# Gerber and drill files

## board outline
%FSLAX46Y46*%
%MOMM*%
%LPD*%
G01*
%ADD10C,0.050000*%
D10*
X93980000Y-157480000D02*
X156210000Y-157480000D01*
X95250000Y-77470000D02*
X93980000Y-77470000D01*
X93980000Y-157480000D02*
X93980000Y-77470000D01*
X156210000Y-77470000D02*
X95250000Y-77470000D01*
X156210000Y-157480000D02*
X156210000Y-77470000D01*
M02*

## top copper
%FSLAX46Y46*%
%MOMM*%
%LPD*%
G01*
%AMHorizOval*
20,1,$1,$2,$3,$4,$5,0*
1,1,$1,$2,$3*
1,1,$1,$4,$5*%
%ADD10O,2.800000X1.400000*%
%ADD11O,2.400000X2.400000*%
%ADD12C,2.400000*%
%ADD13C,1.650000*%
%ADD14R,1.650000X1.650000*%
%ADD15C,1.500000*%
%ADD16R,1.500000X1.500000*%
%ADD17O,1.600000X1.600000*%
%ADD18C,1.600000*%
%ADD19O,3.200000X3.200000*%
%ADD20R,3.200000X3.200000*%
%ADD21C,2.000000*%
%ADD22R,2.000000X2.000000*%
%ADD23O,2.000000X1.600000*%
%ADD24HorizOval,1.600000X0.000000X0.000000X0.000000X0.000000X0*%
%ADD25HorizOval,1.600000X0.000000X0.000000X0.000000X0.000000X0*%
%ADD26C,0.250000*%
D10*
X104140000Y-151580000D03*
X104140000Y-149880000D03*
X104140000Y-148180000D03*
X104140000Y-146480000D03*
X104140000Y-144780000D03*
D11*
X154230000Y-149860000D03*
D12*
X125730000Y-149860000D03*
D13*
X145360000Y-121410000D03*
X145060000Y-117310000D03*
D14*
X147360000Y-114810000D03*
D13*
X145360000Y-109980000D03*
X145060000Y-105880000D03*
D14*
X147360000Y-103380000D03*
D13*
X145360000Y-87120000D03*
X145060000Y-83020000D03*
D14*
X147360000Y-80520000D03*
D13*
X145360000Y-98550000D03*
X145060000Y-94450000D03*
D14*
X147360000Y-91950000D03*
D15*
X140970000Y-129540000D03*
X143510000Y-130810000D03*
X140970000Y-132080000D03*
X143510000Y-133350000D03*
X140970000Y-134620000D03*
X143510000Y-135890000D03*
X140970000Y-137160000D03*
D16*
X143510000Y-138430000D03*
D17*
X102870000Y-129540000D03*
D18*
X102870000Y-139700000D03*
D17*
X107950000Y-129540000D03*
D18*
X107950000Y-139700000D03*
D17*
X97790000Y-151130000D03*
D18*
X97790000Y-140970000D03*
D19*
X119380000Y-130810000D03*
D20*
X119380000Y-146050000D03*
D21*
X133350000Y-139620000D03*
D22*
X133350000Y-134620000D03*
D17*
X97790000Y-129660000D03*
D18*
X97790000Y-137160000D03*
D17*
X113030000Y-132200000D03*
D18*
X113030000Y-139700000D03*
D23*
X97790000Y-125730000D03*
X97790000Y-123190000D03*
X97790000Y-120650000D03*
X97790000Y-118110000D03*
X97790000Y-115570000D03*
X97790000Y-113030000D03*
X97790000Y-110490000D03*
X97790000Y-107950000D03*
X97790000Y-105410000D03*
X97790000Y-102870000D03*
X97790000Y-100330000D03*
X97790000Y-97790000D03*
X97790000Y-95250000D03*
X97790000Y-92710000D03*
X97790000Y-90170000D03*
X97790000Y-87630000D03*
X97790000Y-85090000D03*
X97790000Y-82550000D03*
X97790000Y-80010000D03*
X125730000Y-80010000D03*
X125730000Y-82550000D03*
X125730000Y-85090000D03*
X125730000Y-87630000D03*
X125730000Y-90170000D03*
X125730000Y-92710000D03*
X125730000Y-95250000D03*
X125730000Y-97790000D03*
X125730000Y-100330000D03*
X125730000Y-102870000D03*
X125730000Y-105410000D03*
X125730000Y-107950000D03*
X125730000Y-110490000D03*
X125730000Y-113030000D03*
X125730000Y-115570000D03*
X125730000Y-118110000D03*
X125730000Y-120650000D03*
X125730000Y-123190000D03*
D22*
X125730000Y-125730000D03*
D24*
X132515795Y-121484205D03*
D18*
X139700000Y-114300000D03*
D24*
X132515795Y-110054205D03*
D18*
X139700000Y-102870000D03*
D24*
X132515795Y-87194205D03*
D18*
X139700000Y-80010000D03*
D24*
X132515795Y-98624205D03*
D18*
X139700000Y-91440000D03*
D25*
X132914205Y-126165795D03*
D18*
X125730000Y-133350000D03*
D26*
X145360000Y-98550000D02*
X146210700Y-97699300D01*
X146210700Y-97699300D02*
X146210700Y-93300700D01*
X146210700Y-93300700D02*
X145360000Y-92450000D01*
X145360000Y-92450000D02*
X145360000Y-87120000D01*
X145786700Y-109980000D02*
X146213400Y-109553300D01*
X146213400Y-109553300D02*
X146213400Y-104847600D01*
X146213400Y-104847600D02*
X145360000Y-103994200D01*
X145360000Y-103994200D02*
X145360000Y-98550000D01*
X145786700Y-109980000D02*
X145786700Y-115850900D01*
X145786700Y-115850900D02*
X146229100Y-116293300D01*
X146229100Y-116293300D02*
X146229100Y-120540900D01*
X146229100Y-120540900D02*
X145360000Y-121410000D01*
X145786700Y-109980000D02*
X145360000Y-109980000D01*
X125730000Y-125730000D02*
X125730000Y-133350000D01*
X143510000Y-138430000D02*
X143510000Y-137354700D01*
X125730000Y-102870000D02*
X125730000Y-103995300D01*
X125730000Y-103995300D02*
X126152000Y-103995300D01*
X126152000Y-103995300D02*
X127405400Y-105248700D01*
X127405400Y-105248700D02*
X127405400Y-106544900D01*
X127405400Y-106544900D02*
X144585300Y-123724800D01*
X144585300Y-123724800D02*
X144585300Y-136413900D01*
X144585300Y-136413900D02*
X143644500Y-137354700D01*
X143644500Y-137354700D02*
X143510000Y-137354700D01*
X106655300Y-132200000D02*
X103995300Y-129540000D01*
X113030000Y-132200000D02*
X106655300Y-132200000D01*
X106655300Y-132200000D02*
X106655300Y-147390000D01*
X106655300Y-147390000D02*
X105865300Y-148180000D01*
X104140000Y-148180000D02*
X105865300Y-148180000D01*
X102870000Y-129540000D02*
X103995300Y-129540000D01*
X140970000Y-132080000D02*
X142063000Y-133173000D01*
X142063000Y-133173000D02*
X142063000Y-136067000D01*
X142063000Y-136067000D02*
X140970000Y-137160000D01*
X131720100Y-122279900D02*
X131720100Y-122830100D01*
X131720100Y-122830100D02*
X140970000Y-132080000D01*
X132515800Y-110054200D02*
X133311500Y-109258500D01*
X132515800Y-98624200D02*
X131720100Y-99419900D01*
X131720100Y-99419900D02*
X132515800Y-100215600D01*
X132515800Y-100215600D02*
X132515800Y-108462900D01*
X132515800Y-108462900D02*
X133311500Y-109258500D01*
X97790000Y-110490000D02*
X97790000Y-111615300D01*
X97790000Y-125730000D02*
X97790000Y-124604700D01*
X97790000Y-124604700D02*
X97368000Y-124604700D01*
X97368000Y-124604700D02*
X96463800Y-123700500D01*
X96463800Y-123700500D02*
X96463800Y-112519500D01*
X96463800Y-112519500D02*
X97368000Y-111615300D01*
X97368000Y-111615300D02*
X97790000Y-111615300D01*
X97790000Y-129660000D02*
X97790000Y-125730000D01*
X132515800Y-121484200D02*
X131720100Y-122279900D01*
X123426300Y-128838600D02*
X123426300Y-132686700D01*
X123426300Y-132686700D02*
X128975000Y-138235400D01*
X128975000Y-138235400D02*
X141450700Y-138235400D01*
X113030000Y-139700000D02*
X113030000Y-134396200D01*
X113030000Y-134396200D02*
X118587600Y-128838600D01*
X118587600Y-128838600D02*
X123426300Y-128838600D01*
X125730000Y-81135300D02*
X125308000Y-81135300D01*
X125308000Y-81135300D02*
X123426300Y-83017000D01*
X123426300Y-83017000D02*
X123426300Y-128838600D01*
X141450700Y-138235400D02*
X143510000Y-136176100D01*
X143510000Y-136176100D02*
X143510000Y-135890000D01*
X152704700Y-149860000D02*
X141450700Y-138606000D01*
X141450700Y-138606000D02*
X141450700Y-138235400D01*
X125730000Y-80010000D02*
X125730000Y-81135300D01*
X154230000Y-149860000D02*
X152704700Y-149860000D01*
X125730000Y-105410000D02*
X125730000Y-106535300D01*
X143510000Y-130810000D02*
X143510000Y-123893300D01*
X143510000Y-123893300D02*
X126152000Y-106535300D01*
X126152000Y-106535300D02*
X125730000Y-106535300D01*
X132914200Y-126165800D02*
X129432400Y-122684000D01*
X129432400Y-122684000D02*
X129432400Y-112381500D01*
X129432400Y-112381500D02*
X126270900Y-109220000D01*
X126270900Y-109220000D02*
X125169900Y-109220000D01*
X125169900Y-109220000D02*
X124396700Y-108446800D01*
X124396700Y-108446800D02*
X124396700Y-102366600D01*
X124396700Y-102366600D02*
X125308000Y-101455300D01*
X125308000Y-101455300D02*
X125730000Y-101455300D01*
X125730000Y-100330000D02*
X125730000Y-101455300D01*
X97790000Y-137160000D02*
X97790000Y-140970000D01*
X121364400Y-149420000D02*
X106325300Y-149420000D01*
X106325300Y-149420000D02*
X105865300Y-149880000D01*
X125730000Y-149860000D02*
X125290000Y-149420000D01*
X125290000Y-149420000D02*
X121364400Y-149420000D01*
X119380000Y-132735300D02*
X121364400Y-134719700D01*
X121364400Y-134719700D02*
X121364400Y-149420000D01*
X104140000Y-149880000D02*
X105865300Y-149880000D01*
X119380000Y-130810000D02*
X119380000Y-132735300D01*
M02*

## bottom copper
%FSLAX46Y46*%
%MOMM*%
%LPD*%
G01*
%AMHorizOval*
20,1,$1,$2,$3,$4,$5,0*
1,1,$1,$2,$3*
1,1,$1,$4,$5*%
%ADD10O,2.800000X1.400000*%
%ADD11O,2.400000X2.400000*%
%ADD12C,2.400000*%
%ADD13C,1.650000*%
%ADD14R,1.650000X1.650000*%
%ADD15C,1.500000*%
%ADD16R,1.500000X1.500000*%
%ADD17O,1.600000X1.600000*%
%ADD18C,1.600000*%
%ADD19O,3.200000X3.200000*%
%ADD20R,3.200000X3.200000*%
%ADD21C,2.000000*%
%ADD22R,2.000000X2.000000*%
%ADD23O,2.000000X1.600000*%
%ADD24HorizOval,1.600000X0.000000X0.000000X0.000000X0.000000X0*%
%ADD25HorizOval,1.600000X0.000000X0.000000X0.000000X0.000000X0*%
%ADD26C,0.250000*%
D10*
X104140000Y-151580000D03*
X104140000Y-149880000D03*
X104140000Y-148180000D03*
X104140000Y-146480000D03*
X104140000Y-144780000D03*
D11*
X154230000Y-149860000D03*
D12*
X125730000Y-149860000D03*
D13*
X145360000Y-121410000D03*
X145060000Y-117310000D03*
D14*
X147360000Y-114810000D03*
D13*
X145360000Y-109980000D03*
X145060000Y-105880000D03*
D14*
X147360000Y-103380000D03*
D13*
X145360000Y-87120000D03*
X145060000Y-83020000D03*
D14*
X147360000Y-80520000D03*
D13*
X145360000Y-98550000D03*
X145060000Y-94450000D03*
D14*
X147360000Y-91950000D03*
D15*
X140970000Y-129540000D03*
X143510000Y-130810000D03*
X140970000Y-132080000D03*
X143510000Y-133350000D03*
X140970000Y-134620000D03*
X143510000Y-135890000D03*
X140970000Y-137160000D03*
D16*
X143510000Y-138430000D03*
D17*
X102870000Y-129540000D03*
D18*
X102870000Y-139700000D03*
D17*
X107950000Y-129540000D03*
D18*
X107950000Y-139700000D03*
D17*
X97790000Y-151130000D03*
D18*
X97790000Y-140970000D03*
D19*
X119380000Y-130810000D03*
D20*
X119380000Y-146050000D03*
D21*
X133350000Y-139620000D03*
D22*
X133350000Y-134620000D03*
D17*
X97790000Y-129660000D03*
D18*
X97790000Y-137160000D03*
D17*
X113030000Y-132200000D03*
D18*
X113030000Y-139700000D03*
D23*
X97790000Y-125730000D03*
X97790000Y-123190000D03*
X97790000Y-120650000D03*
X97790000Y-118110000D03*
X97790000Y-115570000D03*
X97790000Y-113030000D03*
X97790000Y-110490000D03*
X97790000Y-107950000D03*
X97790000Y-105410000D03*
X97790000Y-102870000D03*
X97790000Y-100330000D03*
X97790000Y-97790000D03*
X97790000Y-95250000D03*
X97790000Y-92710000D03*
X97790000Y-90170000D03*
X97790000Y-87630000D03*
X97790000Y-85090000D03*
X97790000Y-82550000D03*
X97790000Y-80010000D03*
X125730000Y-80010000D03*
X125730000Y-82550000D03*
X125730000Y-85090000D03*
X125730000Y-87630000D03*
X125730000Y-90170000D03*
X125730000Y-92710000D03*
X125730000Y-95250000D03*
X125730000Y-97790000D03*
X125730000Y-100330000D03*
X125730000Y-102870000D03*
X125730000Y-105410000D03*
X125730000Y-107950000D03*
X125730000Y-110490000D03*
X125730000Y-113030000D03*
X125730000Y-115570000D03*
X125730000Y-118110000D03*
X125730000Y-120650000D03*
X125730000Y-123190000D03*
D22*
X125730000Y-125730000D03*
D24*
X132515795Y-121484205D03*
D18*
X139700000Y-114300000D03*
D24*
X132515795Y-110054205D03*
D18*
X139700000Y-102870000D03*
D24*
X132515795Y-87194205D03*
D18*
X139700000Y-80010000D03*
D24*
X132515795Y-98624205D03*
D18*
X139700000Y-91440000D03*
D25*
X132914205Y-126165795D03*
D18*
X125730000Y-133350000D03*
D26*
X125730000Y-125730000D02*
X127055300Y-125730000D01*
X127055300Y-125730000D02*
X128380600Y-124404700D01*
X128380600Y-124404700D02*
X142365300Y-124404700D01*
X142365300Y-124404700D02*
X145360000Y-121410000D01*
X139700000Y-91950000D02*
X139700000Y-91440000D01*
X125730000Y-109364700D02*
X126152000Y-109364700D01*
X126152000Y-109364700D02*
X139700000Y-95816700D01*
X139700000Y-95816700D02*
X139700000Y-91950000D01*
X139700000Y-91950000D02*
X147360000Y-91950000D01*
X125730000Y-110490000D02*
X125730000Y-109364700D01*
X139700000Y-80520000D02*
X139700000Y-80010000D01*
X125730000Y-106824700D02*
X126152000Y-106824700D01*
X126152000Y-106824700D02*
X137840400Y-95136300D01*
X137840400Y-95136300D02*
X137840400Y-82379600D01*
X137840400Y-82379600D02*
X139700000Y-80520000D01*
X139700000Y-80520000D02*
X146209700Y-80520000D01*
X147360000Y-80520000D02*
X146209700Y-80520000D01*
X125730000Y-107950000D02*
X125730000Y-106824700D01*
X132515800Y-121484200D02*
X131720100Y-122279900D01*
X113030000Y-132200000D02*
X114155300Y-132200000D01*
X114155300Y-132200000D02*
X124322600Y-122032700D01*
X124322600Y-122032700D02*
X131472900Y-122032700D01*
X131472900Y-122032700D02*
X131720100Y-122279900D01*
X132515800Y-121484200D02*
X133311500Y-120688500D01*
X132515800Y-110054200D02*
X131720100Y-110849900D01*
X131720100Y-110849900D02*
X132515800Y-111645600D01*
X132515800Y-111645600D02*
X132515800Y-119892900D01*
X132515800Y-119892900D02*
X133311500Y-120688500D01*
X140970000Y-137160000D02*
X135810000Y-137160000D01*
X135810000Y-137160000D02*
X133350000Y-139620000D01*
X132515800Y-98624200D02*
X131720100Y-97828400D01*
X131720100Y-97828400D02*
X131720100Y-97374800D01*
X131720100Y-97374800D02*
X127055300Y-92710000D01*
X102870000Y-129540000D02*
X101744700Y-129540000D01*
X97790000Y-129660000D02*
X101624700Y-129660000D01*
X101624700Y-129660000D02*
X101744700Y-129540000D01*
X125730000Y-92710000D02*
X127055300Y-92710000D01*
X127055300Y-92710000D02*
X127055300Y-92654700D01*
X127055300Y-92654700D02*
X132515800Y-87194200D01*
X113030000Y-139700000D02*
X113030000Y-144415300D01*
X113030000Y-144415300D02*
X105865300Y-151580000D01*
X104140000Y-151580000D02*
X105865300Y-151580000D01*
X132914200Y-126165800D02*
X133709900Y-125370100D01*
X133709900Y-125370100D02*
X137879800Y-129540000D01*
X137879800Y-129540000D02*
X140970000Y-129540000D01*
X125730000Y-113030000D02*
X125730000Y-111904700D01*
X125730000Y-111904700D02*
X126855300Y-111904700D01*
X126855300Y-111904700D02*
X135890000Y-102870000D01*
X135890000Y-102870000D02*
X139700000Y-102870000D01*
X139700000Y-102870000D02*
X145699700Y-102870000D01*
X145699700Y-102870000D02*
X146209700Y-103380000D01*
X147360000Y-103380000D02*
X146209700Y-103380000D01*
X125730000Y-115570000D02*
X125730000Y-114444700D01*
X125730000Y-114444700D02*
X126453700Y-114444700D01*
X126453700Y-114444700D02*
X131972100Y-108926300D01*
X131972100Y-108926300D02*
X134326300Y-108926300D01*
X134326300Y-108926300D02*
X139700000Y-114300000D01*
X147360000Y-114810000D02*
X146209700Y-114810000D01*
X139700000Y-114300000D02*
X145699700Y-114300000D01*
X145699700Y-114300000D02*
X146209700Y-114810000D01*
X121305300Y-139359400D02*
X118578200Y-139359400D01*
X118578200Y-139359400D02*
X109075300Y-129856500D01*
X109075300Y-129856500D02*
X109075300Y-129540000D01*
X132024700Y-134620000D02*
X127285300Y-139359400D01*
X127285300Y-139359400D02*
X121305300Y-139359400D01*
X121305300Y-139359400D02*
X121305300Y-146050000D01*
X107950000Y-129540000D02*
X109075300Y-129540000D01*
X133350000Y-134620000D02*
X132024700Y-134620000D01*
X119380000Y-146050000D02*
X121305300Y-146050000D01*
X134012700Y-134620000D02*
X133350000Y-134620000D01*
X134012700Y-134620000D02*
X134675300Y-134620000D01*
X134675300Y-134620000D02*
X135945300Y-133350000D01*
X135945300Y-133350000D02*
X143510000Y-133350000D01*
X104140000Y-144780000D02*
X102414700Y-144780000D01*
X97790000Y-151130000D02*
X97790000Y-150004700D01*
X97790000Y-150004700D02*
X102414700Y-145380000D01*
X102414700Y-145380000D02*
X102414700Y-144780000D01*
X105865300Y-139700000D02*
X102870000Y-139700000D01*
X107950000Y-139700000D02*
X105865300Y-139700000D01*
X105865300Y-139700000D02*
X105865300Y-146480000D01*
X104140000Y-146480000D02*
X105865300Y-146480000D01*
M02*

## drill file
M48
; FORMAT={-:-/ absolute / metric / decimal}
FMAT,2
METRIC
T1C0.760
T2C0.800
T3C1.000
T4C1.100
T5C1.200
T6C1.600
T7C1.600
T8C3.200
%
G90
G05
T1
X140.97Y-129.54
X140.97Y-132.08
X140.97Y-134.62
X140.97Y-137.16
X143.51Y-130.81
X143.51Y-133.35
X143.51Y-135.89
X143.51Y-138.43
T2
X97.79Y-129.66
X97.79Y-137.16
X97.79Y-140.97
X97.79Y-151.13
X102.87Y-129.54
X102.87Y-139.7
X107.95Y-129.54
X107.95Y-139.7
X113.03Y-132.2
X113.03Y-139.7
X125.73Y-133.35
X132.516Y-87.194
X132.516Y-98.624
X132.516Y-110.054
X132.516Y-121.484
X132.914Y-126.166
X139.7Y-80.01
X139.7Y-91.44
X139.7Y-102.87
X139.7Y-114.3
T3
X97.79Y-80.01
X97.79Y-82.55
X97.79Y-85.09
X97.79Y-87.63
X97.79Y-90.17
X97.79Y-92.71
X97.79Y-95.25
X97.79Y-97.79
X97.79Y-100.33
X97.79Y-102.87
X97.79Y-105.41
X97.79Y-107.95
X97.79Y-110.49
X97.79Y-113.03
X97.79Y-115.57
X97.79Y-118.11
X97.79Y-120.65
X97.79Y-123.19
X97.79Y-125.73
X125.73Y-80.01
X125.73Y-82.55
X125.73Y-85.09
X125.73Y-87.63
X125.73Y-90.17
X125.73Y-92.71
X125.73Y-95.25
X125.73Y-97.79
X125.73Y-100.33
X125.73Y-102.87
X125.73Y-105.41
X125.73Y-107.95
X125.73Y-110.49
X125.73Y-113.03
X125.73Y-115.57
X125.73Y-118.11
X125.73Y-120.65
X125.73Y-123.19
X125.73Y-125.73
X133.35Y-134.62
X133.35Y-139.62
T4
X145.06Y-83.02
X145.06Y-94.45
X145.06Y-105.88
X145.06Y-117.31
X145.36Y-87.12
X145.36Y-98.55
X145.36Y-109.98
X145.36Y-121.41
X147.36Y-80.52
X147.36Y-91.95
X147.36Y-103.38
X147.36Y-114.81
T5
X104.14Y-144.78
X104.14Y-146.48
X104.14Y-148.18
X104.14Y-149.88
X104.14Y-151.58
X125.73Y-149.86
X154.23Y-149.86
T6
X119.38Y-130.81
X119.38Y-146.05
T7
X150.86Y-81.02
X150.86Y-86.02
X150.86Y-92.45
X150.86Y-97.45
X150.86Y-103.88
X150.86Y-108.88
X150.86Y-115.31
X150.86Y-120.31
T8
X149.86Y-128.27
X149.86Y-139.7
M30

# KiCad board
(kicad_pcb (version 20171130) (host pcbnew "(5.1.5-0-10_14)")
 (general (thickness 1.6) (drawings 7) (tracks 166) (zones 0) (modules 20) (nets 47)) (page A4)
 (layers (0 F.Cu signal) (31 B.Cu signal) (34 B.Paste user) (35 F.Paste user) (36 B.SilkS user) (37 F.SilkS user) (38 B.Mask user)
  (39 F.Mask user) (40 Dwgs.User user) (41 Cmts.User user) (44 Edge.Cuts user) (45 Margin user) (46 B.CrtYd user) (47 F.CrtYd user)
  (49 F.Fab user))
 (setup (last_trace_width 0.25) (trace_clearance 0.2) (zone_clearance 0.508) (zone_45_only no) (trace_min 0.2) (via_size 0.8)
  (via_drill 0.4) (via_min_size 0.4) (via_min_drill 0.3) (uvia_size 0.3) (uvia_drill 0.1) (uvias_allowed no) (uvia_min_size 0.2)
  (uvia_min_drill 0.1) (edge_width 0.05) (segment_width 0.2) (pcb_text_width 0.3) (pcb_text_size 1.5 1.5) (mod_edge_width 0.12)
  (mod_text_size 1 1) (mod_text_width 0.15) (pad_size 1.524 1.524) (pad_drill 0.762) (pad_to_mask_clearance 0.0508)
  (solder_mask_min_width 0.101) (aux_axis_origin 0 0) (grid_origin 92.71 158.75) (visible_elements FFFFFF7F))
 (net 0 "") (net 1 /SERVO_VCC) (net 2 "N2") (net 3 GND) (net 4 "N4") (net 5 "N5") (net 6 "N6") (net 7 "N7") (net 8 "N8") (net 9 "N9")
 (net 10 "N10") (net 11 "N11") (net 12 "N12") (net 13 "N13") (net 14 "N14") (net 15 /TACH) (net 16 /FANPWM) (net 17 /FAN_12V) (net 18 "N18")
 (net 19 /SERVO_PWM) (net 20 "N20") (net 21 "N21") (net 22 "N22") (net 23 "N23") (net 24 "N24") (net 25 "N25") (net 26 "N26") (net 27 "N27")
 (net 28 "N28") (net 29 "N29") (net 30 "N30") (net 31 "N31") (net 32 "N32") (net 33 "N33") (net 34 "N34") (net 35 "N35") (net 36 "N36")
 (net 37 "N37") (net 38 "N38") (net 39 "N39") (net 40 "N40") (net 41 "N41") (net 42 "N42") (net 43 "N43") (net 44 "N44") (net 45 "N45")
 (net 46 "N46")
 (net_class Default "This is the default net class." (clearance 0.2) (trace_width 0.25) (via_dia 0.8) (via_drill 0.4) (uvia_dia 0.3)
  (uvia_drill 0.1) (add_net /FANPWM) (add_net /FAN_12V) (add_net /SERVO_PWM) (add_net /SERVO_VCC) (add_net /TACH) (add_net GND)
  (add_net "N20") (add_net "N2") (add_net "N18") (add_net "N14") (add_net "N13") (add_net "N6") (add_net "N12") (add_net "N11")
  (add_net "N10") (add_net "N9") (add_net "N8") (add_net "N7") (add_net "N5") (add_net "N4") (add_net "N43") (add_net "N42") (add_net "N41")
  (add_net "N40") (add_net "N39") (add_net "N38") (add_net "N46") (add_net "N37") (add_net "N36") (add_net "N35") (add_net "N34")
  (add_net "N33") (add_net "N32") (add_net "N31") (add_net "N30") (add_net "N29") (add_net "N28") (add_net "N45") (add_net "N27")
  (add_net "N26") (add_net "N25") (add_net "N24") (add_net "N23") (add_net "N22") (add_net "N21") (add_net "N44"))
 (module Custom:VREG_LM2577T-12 (layer F.Cu) (at 104.14 144.78 270)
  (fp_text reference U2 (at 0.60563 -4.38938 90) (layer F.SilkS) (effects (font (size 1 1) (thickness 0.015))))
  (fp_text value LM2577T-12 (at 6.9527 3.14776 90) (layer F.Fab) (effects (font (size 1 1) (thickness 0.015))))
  (pad 5 thru_hole oval (at 6.8 0 270) (size 1.4 2.8) (drill 1.2) (layers *.Cu *.Mask) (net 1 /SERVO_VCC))
  (pad 4 thru_hole oval (at 5.1 0 270) (size 1.4 2.8) (drill 1.2) (layers *.Cu *.Mask) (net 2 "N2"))
  (pad 3 thru_hole oval (at 3.4 0 270) (size 1.4 2.8) (drill 1.2) (layers *.Cu *.Mask) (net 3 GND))
  (pad 2 thru_hole oval (at 1.7 0 270) (size 1.4 2.8) (drill 1.2) (layers *.Cu *.Mask) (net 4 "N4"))
  (pad 1 thru_hole oval (at 0 0 270) (size 1.4 2.8) (drill 1.2) (layers *.Cu *.Mask) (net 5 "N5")))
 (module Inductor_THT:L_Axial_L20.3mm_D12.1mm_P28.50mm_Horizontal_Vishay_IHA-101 (layer F.Cu) (at 125.73 149.86)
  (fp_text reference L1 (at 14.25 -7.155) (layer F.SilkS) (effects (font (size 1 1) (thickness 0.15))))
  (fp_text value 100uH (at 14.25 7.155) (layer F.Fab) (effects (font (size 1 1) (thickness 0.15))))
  (pad 2 thru_hole oval (at 28.5 0) (size 2.4 2.4) (drill 1.2) (layers *.Cu *.Mask) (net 1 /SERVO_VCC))
  (pad 1 thru_hole circle (at 0 0) (size 2.4 2.4) (drill 1.2) (layers *.Cu *.Mask) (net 2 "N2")))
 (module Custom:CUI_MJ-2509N (layer F.Cu) (at 149.86 118.11)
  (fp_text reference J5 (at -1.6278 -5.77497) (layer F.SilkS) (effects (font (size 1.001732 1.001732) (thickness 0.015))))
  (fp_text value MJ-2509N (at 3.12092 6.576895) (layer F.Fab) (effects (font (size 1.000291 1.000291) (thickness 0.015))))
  (pad None np_thru_hole circle (at 1 -2.8) (size 1.6 1.6) (drill 1.6) (layers *.Cu *.Mask))
  (pad None np_thru_hole circle (at 1 2.2) (size 1.6 1.6) (drill 1.6) (layers *.Cu *.Mask))
  (pad 3 thru_hole circle (at -4.5 3.3) (size 1.65 1.65) (drill 1.1) (layers *.Cu *.Mask) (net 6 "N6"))
  (pad 2 thru_hole circle (at -4.8 -0.8) (size 1.65 1.65) (drill 1.1) (layers *.Cu *.Mask) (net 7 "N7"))
  (pad 1 thru_hole rect (at -2.5 -3.3) (size 1.65 1.65) (drill 1.1) (layers *.Cu *.Mask) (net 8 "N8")))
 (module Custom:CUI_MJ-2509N (layer F.Cu) (at 149.86 106.68)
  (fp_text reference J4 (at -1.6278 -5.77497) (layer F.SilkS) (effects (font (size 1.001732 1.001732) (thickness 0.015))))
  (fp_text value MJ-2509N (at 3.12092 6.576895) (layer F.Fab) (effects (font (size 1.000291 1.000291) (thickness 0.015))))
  (pad None np_thru_hole circle (at 1 -2.8) (size 1.6 1.6) (drill 1.6) (layers *.Cu *.Mask))
  (pad None np_thru_hole circle (at 1 2.2) (size 1.6 1.6) (drill 1.6) (layers *.Cu *.Mask))
  (pad 3 thru_hole circle (at -4.5 3.3) (size 1.65 1.65) (drill 1.1) (layers *.Cu *.Mask) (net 6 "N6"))
  (pad 2 thru_hole circle (at -4.8 -0.8) (size 1.65 1.65) (drill 1.1) (layers *.Cu *.Mask) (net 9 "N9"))
  (pad 1 thru_hole rect (at -2.5 -3.3) (size 1.65 1.65) (drill 1.1) (layers *.Cu *.Mask) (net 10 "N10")))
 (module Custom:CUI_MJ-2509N (layer F.Cu) (at 149.86 83.82)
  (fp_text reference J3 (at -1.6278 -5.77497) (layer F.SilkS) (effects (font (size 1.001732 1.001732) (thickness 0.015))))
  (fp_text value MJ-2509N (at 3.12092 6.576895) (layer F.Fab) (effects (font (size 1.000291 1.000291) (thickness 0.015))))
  (pad None np_thru_hole circle (at 1 -2.8) (size 1.6 1.6) (drill 1.6) (layers *.Cu *.Mask))
  (pad None np_thru_hole circle (at 1 2.2) (size 1.6 1.6) (drill 1.6) (layers *.Cu *.Mask))
  (pad 3 thru_hole circle (at -4.5 3.3) (size 1.65 1.65) (drill 1.1) (layers *.Cu *.Mask) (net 6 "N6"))
  (pad 2 thru_hole circle (at -4.8 -0.8) (size 1.65 1.65) (drill 1.1) (layers *.Cu *.Mask) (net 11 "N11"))
  (pad 1 thru_hole rect (at -2.5 -3.3) (size 1.65 1.65) (drill 1.1) (layers *.Cu *.Mask) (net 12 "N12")))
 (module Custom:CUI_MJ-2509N (layer F.Cu) (at 149.86 95.25)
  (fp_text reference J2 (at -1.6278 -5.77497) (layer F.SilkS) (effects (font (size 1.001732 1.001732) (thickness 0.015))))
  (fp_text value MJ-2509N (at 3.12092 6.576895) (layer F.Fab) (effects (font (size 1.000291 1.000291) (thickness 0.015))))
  (pad None np_thru_hole circle (at 1 -2.8) (size 1.6 1.6) (drill 1.6) (layers *.Cu *.Mask))
  (pad None np_thru_hole circle (at 1 2.2) (size 1.6 1.6) (drill 1.6) (layers *.Cu *.Mask))
  (pad 3 thru_hole circle (at -4.5 3.3) (size 1.65 1.65) (drill 1.1) (layers *.Cu *.Mask) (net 6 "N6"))
  (pad 2 thru_hole circle (at -4.8 -0.8) (size 1.65 1.65) (drill 1.1) (layers *.Cu *.Mask) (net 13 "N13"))
  (pad 1 thru_hole rect (at -2.5 -3.3) (size 1.65 1.65) (drill 1.1) (layers *.Cu *.Mask) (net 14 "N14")))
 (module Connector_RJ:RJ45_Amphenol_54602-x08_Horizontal (layer F.Cu) (at 143.51 138.43 90)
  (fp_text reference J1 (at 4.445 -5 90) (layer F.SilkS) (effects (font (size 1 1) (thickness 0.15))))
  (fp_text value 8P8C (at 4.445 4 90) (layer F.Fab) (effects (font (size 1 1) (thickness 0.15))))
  (pad 8 thru_hole circle (at 8.89 -2.54 90) (size 1.5 1.5) (drill 0.76) (layers *.Cu *.Mask) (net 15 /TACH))
  (pad 7 thru_hole circle (at 7.62 0 90) (size 1.5 1.5) (drill 0.76) (layers *.Cu *.Mask) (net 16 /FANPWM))
  (pad 6 thru_hole circle (at 6.35 -2.54 90) (size 1.5 1.5) (drill 0.76) (layers *.Cu *.Mask) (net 3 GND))
  (pad 5 thru_hole circle (at 5.08 0 90) (size 1.5 1.5) (drill 0.76) (layers *.Cu *.Mask) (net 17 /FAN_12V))
  (pad 4 thru_hole circle (at 3.81 -2.54 90) (size 1.5 1.5) (drill 0.76) (layers *.Cu *.Mask) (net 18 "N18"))
  (pad 3 thru_hole circle (at 2.54 0 90) (size 1.5 1.5) (drill 0.76) (layers *.Cu *.Mask) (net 1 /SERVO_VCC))
  (pad 2 thru_hole circle (at 1.27 -2.54 90) (size 1.5 1.5) (drill 0.76) (layers *.Cu *.Mask) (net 3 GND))
  (pad 1 thru_hole rect (at 0 0 90) (size 1.5 1.5) (drill 0.76) (layers *.Cu *.Mask) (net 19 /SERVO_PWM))
  (pad "" np_thru_hole circle (at -1.27 6.35 90) (size 3.2 3.2) (drill 3.2) (layers *.Cu *.Mask))
  (pad "" np_thru_hole circle (at 10.16 6.35 90) (size 3.2 3.2) (drill 3.2) (layers *.Cu *.Mask)))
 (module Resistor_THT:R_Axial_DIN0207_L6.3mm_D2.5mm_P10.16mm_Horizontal (layer F.Cu) (at 102.87 139.7 90)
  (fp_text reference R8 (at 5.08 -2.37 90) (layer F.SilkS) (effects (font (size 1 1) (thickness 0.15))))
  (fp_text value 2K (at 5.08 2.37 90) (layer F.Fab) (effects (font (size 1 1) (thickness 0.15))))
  (pad 2 thru_hole oval (at 10.16 0 90) (size 1.6 1.6) (drill 0.8) (layers *.Cu *.Mask) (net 3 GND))
  (pad 1 thru_hole circle (at 0 0 90) (size 1.6 1.6) (drill 0.8) (layers *.Cu *.Mask) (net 4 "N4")))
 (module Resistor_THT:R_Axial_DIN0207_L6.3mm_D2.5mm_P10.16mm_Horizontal (layer F.Cu) (at 107.95 139.7 90)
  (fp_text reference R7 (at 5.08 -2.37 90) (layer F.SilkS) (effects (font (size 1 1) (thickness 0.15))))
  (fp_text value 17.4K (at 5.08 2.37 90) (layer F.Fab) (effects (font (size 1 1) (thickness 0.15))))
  (pad 2 thru_hole oval (at 10.16 0 90) (size 1.6 1.6) (drill 0.8) (layers *.Cu *.Mask) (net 17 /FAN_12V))
  (pad 1 thru_hole circle (at 0 0 90) (size 1.6 1.6) (drill 0.8) (layers *.Cu *.Mask) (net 4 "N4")))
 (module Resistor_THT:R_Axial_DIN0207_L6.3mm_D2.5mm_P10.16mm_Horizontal (layer F.Cu) (at 97.79 140.97 270)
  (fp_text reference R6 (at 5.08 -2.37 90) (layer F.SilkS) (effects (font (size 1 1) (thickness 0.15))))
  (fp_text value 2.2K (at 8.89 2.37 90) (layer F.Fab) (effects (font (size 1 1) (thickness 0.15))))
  (pad 2 thru_hole oval (at 10.16 0 270) (size 1.6 1.6) (drill 0.8) (layers *.Cu *.Mask) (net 5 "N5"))
  (pad 1 thru_hole circle (at 0 0 270) (size 1.6 1.6) (drill 0.8) (layers *.Cu *.Mask) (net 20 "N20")))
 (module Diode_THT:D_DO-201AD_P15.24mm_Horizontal (layer F.Cu) (at 119.38 146.05 90)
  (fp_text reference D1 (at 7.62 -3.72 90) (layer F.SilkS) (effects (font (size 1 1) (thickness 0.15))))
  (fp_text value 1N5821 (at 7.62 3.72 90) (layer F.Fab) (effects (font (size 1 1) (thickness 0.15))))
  (pad 2 thru_hole oval (at 15.24 0 90) (size 3.2 3.2) (drill 1.6) (layers *.Cu *.Mask) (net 2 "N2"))
  (pad 1 thru_hole rect (at 0 0 90) (size 3.2 3.2) (drill 1.6) (layers *.Cu *.Mask) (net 17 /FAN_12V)))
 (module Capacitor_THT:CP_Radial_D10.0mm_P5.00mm (layer F.Cu) (at 133.35 134.62 270)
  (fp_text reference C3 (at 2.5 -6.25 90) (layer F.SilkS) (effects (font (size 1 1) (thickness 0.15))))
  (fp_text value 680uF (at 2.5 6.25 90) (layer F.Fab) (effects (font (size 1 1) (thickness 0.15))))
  (pad 2 thru_hole circle (at 5 0 270) (size 2 2) (drill 1) (layers *.Cu *.Mask) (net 3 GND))
  (pad 1 thru_hole rect (at 0 0 270) (size 2 2) (drill 1) (layers *.Cu *.Mask) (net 17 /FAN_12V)))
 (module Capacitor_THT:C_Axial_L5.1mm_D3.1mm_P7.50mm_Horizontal (layer F.Cu) (at 97.79 137.16 90)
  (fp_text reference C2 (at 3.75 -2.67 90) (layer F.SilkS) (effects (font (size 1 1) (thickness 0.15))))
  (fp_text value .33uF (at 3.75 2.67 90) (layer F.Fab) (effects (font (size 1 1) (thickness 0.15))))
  (pad 2 thru_hole oval (at 7.5 0 90) (size 1.6 1.6) (drill 0.8) (layers *.Cu *.Mask) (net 3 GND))
  (pad 1 thru_hole circle (at 0 0 90) (size 1.6 1.6) (drill 0.8) (layers *.Cu *.Mask) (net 20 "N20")))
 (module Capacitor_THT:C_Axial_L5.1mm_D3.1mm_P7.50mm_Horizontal (layer F.Cu) (at 113.03 139.7 90)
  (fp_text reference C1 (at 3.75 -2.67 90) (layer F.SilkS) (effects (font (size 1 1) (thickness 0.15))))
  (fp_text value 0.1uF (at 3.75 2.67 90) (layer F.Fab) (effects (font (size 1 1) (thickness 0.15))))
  (pad 2 thru_hole oval (at 7.5 0 90) (size 1.6 1.6) (drill 0.8) (layers *.Cu *.Mask) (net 3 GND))
  (pad 1 thru_hole circle (at 0 0 90) (size 1.6 1.6) (drill 0.8) (layers *.Cu *.Mask) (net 1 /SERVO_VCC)))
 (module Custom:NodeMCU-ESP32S (layer F.Cu) (at 125.73 125.73 180)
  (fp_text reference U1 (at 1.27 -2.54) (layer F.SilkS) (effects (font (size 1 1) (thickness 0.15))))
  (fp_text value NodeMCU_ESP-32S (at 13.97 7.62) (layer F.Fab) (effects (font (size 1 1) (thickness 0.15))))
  (pad 38 thru_hole oval (at 27.94 0 180) (size 2 1.6) (drill 1) (layers *.Cu *.Mask) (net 3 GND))
  (pad 37 thru_hole oval (at 27.94 2.54 180) (size 2 1.6) (drill 1) (layers *.Cu *.Mask) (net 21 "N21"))
  (pad 36 thru_hole oval (at 27.94 5.08 180) (size 2 1.6) (drill 1) (layers *.Cu *.Mask) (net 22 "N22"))
  (pad 35 thru_hole oval (at 27.94 7.62 180) (size 2 1.6) (drill 1) (layers *.Cu *.Mask) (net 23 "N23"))
  (pad 34 thru_hole oval (at 27.94 10.16 180) (size 2 1.6) (drill 1) (layers *.Cu *.Mask) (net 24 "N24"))
  (pad 33 thru_hole oval (at 27.94 12.7 180) (size 2 1.6) (drill 1) (layers *.Cu *.Mask) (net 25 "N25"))
  (pad 32 thru_hole oval (at 27.94 15.24 180) (size 2 1.6) (drill 1) (layers *.Cu *.Mask) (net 3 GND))
  (pad 31 thru_hole oval (at 27.94 17.78 180) (size 2 1.6) (drill 1) (layers *.Cu *.Mask) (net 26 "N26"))
  (pad 30 thru_hole oval (at 27.94 20.32 180) (size 2 1.6) (drill 1) (layers *.Cu *.Mask) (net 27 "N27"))
  (pad 29 thru_hole oval (at 27.94 22.86 180) (size 2 1.6) (drill 1) (layers *.Cu *.Mask) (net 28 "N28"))
  (pad 28 thru_hole oval (at 27.94 25.4 180) (size 2 1.6) (drill 1) (layers *.Cu *.Mask) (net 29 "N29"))
  (pad 27 thru_hole oval (at 27.94 27.94 180) (size 2 1.6) (drill 1) (layers *.Cu *.Mask) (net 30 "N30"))
  (pad 26 thru_hole oval (at 27.94 30.48 180) (size 2 1.6) (drill 1) (layers *.Cu *.Mask) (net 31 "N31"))
  (pad 25 thru_hole oval (at 27.94 33.02 180) (size 2 1.6) (drill 1) (layers *.Cu *.Mask) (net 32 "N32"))
  (pad 24 thru_hole oval (at 27.94 35.56 180) (size 2 1.6) (drill 1) (layers *.Cu *.Mask) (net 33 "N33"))
  (pad 23 thru_hole oval (at 27.94 38.1 180) (size 2 1.6) (drill 1) (layers *.Cu *.Mask) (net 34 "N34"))
  (pad 22 thru_hole oval (at 27.94 40.64 180) (size 2 1.6) (drill 1) (layers *.Cu *.Mask) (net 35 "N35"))
  (pad 21 thru_hole oval (at 27.94 43.18 180) (size 2 1.6) (drill 1) (layers *.Cu *.Mask) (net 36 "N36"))
  (pad 20 thru_hole oval (at 27.94 45.72 180) (size 2 1.6) (drill 1) (layers *.Cu *.Mask) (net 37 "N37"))
  (pad 19 thru_hole oval (at 0 45.72 180) (size 2 1.6) (drill 1) (layers *.Cu *.Mask) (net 1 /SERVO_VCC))
  (pad 18 thru_hole oval (at 0 43.18 180) (size 2 1.6) (drill 1) (layers *.Cu *.Mask) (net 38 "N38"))
  (pad 17 thru_hole oval (at 0 40.64 180) (size 2 1.6) (drill 1) (layers *.Cu *.Mask) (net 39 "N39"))
  (pad 16 thru_hole oval (at 0 38.1 180) (size 2 1.6) (drill 1) (layers *.Cu *.Mask) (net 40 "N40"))
  (pad 15 thru_hole oval (at 0 35.56 180) (size 2 1.6) (drill 1) (layers *.Cu *.Mask) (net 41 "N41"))
  (pad 14 thru_hole oval (at 0 33.02 180) (size 2 1.6) (drill 1) (layers *.Cu *.Mask) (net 3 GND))
  (pad 13 thru_hole oval (at 0 30.48 180) (size 2 1.6) (drill 1) (layers *.Cu *.Mask) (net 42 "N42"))
  (pad 12 thru_hole oval (at 0 27.94 180) (size 2 1.6) (drill 1) (layers *.Cu *.Mask) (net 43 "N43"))
  (pad 11 thru_hole oval (at 0 25.4 180) (size 2 1.6) (drill 1) (layers *.Cu *.Mask) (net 15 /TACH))
  (pad 10 thru_hole oval (at 0 22.86 180) (size 2 1.6) (drill 1) (layers *.Cu *.Mask) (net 19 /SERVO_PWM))
  (pad 9 thru_hole oval (at 0 20.32 180) (size 2 1.6) (drill 1) (layers *.Cu *.Mask) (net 16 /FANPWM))
  (pad 8 thru_hole oval (at 0 17.78 180) (size 2 1.6) (drill 1) (layers *.Cu *.Mask) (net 12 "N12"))
  (pad 7 thru_hole oval (at 0 15.24 180) (size 2 1.6) (drill 1) (layers *.Cu *.Mask) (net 14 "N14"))
  (pad 6 thru_hole oval (at 0 12.7 180) (size 2 1.6) (drill 1) (layers *.Cu *.Mask) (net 10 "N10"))
  (pad 5 thru_hole oval (at 0 10.16 180) (size 2 1.6) (drill 1) (layers *.Cu *.Mask) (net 8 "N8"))
  (pad 4 thru_hole oval (at 0 7.62 180) (size 2 1.6) (drill 1) (layers *.Cu *.Mask) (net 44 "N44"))
  (pad 3 thru_hole oval (at 0 5.08 180) (size 2 1.6) (drill 1) (layers *.Cu *.Mask) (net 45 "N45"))
  (pad 2 thru_hole oval (at 0 2.54 180) (size 2 1.6) (drill 1) (layers *.Cu *.Mask) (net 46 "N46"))
  (pad 1 thru_hole rect (at 0 0 180) (size 2 2) (drill 1) (layers *.Cu *.Mask) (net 6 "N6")))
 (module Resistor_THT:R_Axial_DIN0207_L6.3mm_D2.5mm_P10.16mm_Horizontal (layer F.Cu) (at 139.7 114.3 225)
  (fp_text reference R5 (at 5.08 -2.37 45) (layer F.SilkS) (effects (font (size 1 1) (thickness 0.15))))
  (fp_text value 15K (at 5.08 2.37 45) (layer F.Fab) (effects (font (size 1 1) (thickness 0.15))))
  (pad 2 thru_hole oval (at 10.16 0 225) (size 1.6 1.6) (drill 0.8) (layers *.Cu *.Mask) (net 3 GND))
  (pad 1 thru_hole circle (at 0 0 225) (size 1.6 1.6) (drill 0.8) (layers *.Cu *.Mask) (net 8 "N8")))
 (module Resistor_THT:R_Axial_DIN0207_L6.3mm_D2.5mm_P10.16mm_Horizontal (layer F.Cu) (at 139.7 102.87 225)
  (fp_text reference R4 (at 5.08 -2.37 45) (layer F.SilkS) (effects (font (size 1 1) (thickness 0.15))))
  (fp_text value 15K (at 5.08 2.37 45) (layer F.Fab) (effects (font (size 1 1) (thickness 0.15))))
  (pad 2 thru_hole oval (at 10.16 0 225) (size 1.6 1.6) (drill 0.8) (layers *.Cu *.Mask) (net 3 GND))
  (pad 1 thru_hole circle (at 0 0 225) (size 1.6 1.6) (drill 0.8) (layers *.Cu *.Mask) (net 10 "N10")))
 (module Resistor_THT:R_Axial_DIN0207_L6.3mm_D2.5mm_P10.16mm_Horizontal (layer F.Cu) (at 139.7 80.01 225)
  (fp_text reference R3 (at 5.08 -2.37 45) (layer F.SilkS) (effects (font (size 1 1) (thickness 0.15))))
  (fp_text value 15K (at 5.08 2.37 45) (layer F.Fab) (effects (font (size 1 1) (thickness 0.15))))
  (pad 2 thru_hole oval (at 10.16 0 225) (size 1.6 1.6) (drill 0.8) (layers *.Cu *.Mask) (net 3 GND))
  (pad 1 thru_hole circle (at 0 0 225) (size 1.6 1.6) (drill 0.8) (layers *.Cu *.Mask) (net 12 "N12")))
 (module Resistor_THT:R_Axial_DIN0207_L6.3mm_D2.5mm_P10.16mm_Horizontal (layer F.Cu) (at 139.7 91.44 225)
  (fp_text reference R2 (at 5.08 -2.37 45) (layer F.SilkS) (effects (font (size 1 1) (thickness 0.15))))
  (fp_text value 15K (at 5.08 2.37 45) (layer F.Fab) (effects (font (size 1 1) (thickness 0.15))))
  (pad 2 thru_hole oval (at 10.16 0 225) (size 1.6 1.6) (drill 0.8) (layers *.Cu *.Mask) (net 3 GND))
  (pad 1 thru_hole circle (at 0 0 225) (size 1.6 1.6) (drill 0.8) (layers *.Cu *.Mask) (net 14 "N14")))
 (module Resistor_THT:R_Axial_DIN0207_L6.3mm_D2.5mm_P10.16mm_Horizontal (layer F.Cu) (at 125.73 133.35 45)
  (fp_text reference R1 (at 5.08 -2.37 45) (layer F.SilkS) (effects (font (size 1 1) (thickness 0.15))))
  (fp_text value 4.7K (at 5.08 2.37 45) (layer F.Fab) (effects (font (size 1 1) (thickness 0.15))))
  (pad 2 thru_hole oval (at 10.16 0 45) (size 1.6 1.6) (drill 0.8) (layers *.Cu *.Mask) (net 15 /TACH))
  (pad 1 thru_hole circle (at 0 0 45) (size 1.6 1.6) (drill 0.8) (layers *.Cu *.Mask) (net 6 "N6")))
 (gr_line (start 93.98 157.48) (end 156.21 157.48) (layer Edge.Cuts) (width 0.05))
 (gr_line (start 95.25 77.47) (end 93.98 77.47) (layer Edge.Cuts) (width 0.05))
 (gr_line (start 93.98 157.48) (end 93.98 77.47) (layer Edge.Cuts) (width 0.05))
 (gr_line (start 156.21 77.47) (end 95.25 77.47) (layer Edge.Cuts) (width 0.05))
 (gr_line (start 156.21 157.48) (end 156.21 77.47) (layer Edge.Cuts) (width 0.05))
 (segment (start 145.36 98.55) (end 146.2107 97.6993) (width 0.25) (layer F.Cu) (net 6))
 (segment (start 146.2107 97.6993) (end 146.2107 93.3007) (width 0.25) (layer F.Cu) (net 6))
 (segment (start 146.2107 93.3007) (end 145.36 92.45) (width 0.25) (layer F.Cu) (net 6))
 (segment (start 145.36 92.45) (end 145.36 87.12) (width 0.25) (layer F.Cu) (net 6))
 (segment (start 145.7867 109.98) (end 146.2134 109.5533) (width 0.25) (layer F.Cu) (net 6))
 (segment (start 146.2134 109.5533) (end 146.2134 104.8476) (width 0.25) (layer F.Cu) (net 6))
 (segment (start 146.2134 104.8476) (end 145.36 103.9942) (width 0.25) (layer F.Cu) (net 6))
 (segment (start 145.36 103.9942) (end 145.36 98.55) (width 0.25) (layer F.Cu) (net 6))
 (segment (start 125.73 125.73) (end 127.0553 125.73) (width 0.25) (layer B.Cu) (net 6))
 (segment (start 127.0553 125.73) (end 128.3806 124.4047) (width 0.25) (layer B.Cu) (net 6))
 (segment (start 128.3806 124.4047) (end 142.3653 124.4047) (width 0.25) (layer B.Cu) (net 6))
 (segment (start 142.3653 124.4047) (end 145.36 121.41) (width 0.25) (layer B.Cu) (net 6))
 (segment (start 145.7867 109.98) (end 145.7867 115.8509) (width 0.25) (layer F.Cu) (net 6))
 (segment (start 145.7867 115.8509) (end 146.2291 116.2933) (width 0.25) (layer F.Cu) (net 6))
 (segment (start 146.2291 116.2933) (end 146.2291 120.5409) (width 0.25) (layer F.Cu) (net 6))
 (segment (start 146.2291 120.5409) (end 145.36 121.41) (width 0.25) (layer F.Cu) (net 6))
 (segment (start 145.7867 109.98) (end 145.36 109.98) (width 0.25) (layer F.Cu) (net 6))
 (segment (start 125.73 125.73) (end 125.73 133.35) (width 0.25) (layer F.Cu) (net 6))
 (segment (start 139.7 91.95) (end 139.7 91.44) (width 0.25) (layer B.Cu) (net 14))
 (segment (start 125.73 109.3647) (end 126.152 109.3647) (width 0.25) (layer B.Cu) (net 14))
 (segment (start 126.152 109.3647) (end 139.7 95.8167) (width 0.25) (layer B.Cu) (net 14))
 (segment (start 139.7 95.8167) (end 139.7 91.95) (width 0.25) (layer B.Cu) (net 14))
 (segment (start 139.7 91.95) (end 147.36 91.95) (width 0.25) (layer B.Cu) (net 14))
 (segment (start 125.73 110.49) (end 125.73 109.3647) (width 0.25) (layer B.Cu) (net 14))
 (segment (start 139.7 80.52) (end 139.7 80.01) (width 0.25) (layer B.Cu) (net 12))
 (segment (start 125.73 106.8247) (end 126.152 106.8247) (width 0.25) (layer B.Cu) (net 12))
 (segment (start 126.152 106.8247) (end 137.8404 95.1363) (width 0.25) (layer B.Cu) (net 12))
 (segment (start 137.8404 95.1363) (end 137.8404 82.3796) (width 0.25) (layer B.Cu) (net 12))
 (segment (start 137.8404 82.3796) (end 139.7 80.52) (width 0.25) (layer B.Cu) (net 12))
 (segment (start 139.7 80.52) (end 146.2097 80.52) (width 0.25) (layer B.Cu) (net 12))
 (segment (start 147.36 80.52) (end 146.2097 80.52) (width 0.25) (layer B.Cu) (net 12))
 (segment (start 125.73 107.95) (end 125.73 106.8247) (width 0.25) (layer B.Cu) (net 12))
 (segment (start 143.51 138.43) (end 143.51 137.3547) (width 0.25) (layer F.Cu) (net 19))
 (segment (start 125.73 102.87) (end 125.73 103.9953) (width 0.25) (layer F.Cu) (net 19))
 (segment (start 125.73 103.9953) (end 126.152 103.9953) (width 0.25) (layer F.Cu) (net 19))
 (segment (start 126.152 103.9953) (end 127.4054 105.2487) (width 0.25) (layer F.Cu) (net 19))
 (segment (start 127.4054 105.2487) (end 127.4054 106.5449) (width 0.25) (layer F.Cu) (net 19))
 (segment (start 127.4054 106.5449) (end 144.5853 123.7248) (width 0.25) (layer F.Cu) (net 19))
 (segment (start 144.5853 123.7248) (end 144.5853 136.4139) (width 0.25) (layer F.Cu) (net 19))
 (segment (start 144.5853 136.4139) (end 143.6445 137.3547) (width 0.25) (layer F.Cu) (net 19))
 (segment (start 143.6445 137.3547) (end 143.51 137.3547) (width 0.25) (layer F.Cu) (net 19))
 (segment (start 132.5158 121.4842) (end 131.7201 122.2799) (width 0.25) (layer B.Cu) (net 3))
 (segment (start 113.03 132.2) (end 114.1553 132.2) (width 0.25) (layer B.Cu) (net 3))
 (segment (start 114.1553 132.2) (end 124.3226 122.0327) (width 0.25) (layer B.Cu) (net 3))
 (segment (start 124.3226 122.0327) (end 131.4729 122.0327) (width 0.25) (layer B.Cu) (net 3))
 (segment (start 131.4729 122.0327) (end 131.7201 122.2799) (width 0.25) (layer B.Cu) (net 3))
 (segment (start 132.5158 121.4842) (end 133.3115 120.6885) (width 0.25) (layer B.Cu) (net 3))
 (segment (start 132.5158 110.0542) (end 131.7201 110.8499) (width 0.25) (layer B.Cu) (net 3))
 (segment (start 131.7201 110.8499) (end 132.5158 111.6456) (width 0.25) (layer B.Cu) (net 3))
 (segment (start 132.5158 111.6456) (end 132.5158 119.8929) (width 0.25) (layer B.Cu) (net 3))
 (segment (start 132.5158 119.8929) (end 133.3115 120.6885) (width 0.25) (layer B.Cu) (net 3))
 (segment (start 106.6553 132.2) (end 103.9953 129.54) (width 0.25) (layer F.Cu) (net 3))
 (segment (start 113.03 132.2) (end 106.6553 132.2) (width 0.25) (layer F.Cu) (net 3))
 (segment (start 106.6553 132.2) (end 106.6553 147.39) (width 0.25) (layer F.Cu) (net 3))
 (segment (start 106.6553 147.39) (end 105.8653 148.18) (width 0.25) (layer F.Cu) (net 3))
 (segment (start 104.14 148.18) (end 105.8653 148.18) (width 0.25) (layer F.Cu) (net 3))
 (segment (start 102.87 129.54) (end 103.9953 129.54) (width 0.25) (layer F.Cu) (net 3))
 (segment (start 140.97 132.08) (end 142.063 133.173) (width 0.25) (layer F.Cu) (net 3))
 (segment (start 142.063 133.173) (end 142.063 136.067) (width 0.25) (layer F.Cu) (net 3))
 (segment (start 142.063 136.067) (end 140.97 137.16) (width 0.25) (layer F.Cu) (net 3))
 (segment (start 131.7201 122.2799) (end 131.7201 122.8301) (width 0.25) (layer F.Cu) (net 3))
 (segment (start 131.7201 122.8301) (end 140.97 132.08) (width 0.25) (layer F.Cu) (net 3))
 (segment (start 140.97 137.16) (end 135.81 137.16) (width 0.25) (layer B.Cu) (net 3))
 (segment (start 135.81 137.16) (end 133.35 139.62) (width 0.25) (layer B.Cu) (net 3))
 (segment (start 132.5158 110.0542) (end 133.3115 109.2585) (width 0.25) (layer F.Cu) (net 3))
 (segment (start 132.5158 98.6242) (end 131.7201 99.4199) (width 0.25) (layer F.Cu) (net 3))
 (segment (start 131.7201 99.4199) (end 132.5158 100.2156) (width 0.25) (layer F.Cu) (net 3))
 (segment (start 132.5158 100.2156) (end 132.5158 108.4629) (width 0.25) (layer F.Cu) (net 3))
 (segment (start 132.5158 108.4629) (end 133.3115 109.2585) (width 0.25) (layer F.Cu) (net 3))
 (segment (start 97.79 110.49) (end 97.79 111.6153) (width 0.25) (layer F.Cu) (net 3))
 (segment (start 97.79 125.73) (end 97.79 124.6047) (width 0.25) (layer F.Cu) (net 3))
 (segment (start 97.79 124.6047) (end 97.368 124.6047) (width 0.25) (layer F.Cu) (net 3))
 (segment (start 97.368 124.6047) (end 96.4638 123.7005) (width 0.25) (layer F.Cu) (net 3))
 (segment (start 96.4638 123.7005) (end 96.4638 112.5195) (width 0.25) (layer F.Cu) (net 3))
 (segment (start 96.4638 112.5195) (end 97.368 111.6153) (width 0.25) (layer F.Cu) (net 3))
 (segment (start 97.368 111.6153) (end 97.79 111.6153) (width 0.25) (layer F.Cu) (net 3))
 (segment (start 97.79 129.66) (end 97.79 125.73) (width 0.25) (layer F.Cu) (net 3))
 (segment (start 132.5158 121.4842) (end 131.7201 122.2799) (width 0.25) (layer F.Cu) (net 3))
 (segment (start 132.5158 98.6242) (end 131.7201 97.8284) (width 0.25) (layer B.Cu) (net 3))
 (segment (start 131.7201 97.8284) (end 131.7201 97.3748) (width 0.25) (layer B.Cu) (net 3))
 (segment (start 131.7201 97.3748) (end 127.0553 92.71) (width 0.25) (layer B.Cu) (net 3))
 (segment (start 102.87 129.54) (end 101.7447 129.54) (width 0.25) (layer B.Cu) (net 3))
 (segment (start 97.79 129.66) (end 101.6247 129.66) (width 0.25) (layer B.Cu) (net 3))
 (segment (start 101.6247 129.66) (end 101.7447 129.54) (width 0.25) (layer B.Cu) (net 3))
 (segment (start 125.73 92.71) (end 127.0553 92.71) (width 0.25) (layer B.Cu) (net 3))
 (segment (start 127.0553 92.71) (end 127.0553 92.6547) (width 0.25) (layer B.Cu) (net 3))
 (segment (start 127.0553 92.6547) (end 132.5158 87.1942) (width 0.25) (layer B.Cu) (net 3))
 (segment (start 123.4263 128.8386) (end 123.4263 132.6867) (width 0.25) (layer F.Cu) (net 1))
 (segment (start 123.4263 132.6867) (end 128.975 138.2354) (width 0.25) (layer F.Cu) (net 1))
 (segment (start 128.975 138.2354) (end 141.4507 138.2354) (width 0.25) (layer F.Cu) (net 1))
 (segment (start 113.03 139.7) (end 113.03 134.3962) (width 0.25) (layer F.Cu) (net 1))
 (segment (start 113.03 134.3962) (end 118.5876 128.8386) (width 0.25) (layer F.Cu) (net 1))
 (segment (start 118.5876 128.8386) (end 123.4263 128.8386) (width 0.25) (layer F.Cu) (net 1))
 (segment (start 125.73 81.1353) (end 125.308 81.1353) (width 0.25) (layer F.Cu) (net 1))
 (segment (start 125.308 81.1353) (end 123.4263 83.017) (width 0.25) (layer F.Cu) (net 1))
 (segment (start 123.4263 83.017) (end 123.4263 128.8386) (width 0.25) (layer F.Cu) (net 1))
 (segment (start 141.4507 138.2354) (end 143.51 136.1761) (width 0.25) (layer F.Cu) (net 1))
 (segment (start 143.51 136.1761) (end 143.51 135.89) (width 0.25) (layer F.Cu) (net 1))
 (segment (start 152.7047 149.86) (end 141.4507 138.606) (width 0.25) (layer F.Cu) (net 1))
 (segment (start 141.4507 138.606) (end 141.4507 138.2354) (width 0.25) (layer F.Cu) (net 1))
 (segment (start 125.73 80.01) (end 125.73 81.1353) (width 0.25) (layer F.Cu) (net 1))
 (segment (start 154.23 149.86) (end 152.7047 149.86) (width 0.25) (layer F.Cu) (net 1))
 (segment (start 113.03 139.7) (end 113.03 144.4153) (width 0.25) (layer B.Cu) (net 1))
 (segment (start 113.03 144.4153) (end 105.8653 151.58) (width 0.25) (layer B.Cu) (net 1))
 (segment (start 104.14 151.58) (end 105.8653 151.58) (width 0.25) (layer B.Cu) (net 1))
 (segment (start 125.73 105.41) (end 125.73 106.5353) (width 0.25) (layer F.Cu) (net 16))
 (segment (start 143.51 130.81) (end 143.51 123.8933) (width 0.25) (layer F.Cu) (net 16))
 (segment (start 143.51 123.8933) (end 126.152 106.5353) (width 0.25) (layer F.Cu) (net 16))
 (segment (start 126.152 106.5353) (end 125.73 106.5353) (width 0.25) (layer F.Cu) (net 16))
 (segment (start 132.9142 126.1658) (end 129.4324 122.684) (width 0.25) (layer F.Cu) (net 15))
 (segment (start 129.4324 122.684) (end 129.4324 112.3815) (width 0.25) (layer F.Cu) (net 15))
 (segment (start 129.4324 112.3815) (end 126.2709 109.22) (width 0.25) (layer F.Cu) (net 15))
 (segment (start 126.2709 109.22) (end 125.1699 109.22) (width 0.25) (layer F.Cu) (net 15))
 (segment (start 125.1699 109.22) (end 124.3967 108.4468) (width 0.25) (layer F.Cu) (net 15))
 (segment (start 124.3967 108.4468) (end 124.3967 102.3666) (width 0.25) (layer F.Cu) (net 15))
 (segment (start 124.3967 102.3666) (end 125.308 101.4553) (width 0.25) (layer F.Cu) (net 15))
 (segment (start 125.308 101.4553) (end 125.73 101.4553) (width 0.25) (layer F.Cu) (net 15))
 (segment (start 132.9142 126.1658) (end 133.7099 125.3701) (width 0.25) (layer B.Cu) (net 15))
 (segment (start 133.7099 125.3701) (end 137.8798 129.54) (width 0.25) (layer B.Cu) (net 15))
 (segment (start 137.8798 129.54) (end 140.97 129.54) (width 0.25) (layer B.Cu) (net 15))
 (segment (start 125.73 100.33) (end 125.73 101.4553) (width 0.25) (layer F.Cu) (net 15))
 (segment (start 125.73 113.03) (end 125.73 111.9047) (width 0.25) (layer B.Cu) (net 10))
 (segment (start 125.73 111.9047) (end 126.8553 111.9047) (width 0.25) (layer B.Cu) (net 10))
 (segment (start 126.8553 111.9047) (end 135.89 102.87) (width 0.25) (layer B.Cu) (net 10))
 (segment (start 135.89 102.87) (end 139.7 102.87) (width 0.25) (layer B.Cu) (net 10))
 (segment (start 139.7 102.87) (end 145.6997 102.87) (width 0.25) (layer B.Cu) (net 10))
 (segment (start 145.6997 102.87) (end 146.2097 103.38) (width 0.25) (layer B.Cu) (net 10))
 (segment (start 147.36 103.38) (end 146.2097 103.38) (width 0.25) (layer B.Cu) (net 10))
 (segment (start 125.73 115.57) (end 125.73 114.4447) (width 0.25) (layer B.Cu) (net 8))
 (segment (start 125.73 114.4447) (end 126.4537 114.4447) (width 0.25) (layer B.Cu) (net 8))
 (segment (start 126.4537 114.4447) (end 131.9721 108.9263) (width 0.25) (layer B.Cu) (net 8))
 (segment (start 131.9721 108.9263) (end 134.3263 108.9263) (width 0.25) (layer B.Cu) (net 8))
 (segment (start 134.3263 108.9263) (end 139.7 114.3) (width 0.25) (layer B.Cu) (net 8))
 (segment (start 147.36 114.81) (end 146.2097 114.81) (width 0.25) (layer B.Cu) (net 8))
 (segment (start 139.7 114.3) (end 145.6997 114.3) (width 0.25) (layer B.Cu) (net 8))
 (segment (start 145.6997 114.3) (end 146.2097 114.81) (width 0.25) (layer B.Cu) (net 8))
 (segment (start 97.79 137.16) (end 97.79 140.97) (width 0.25) (layer F.Cu) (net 20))
 (segment (start 121.3053 139.3594) (end 118.5782 139.3594) (width 0.25) (layer B.Cu) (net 17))
 (segment (start 118.5782 139.3594) (end 109.0753 129.8565) (width 0.25) (layer B.Cu) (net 17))
 (segment (start 109.0753 129.8565) (end 109.0753 129.54) (width 0.25) (layer B.Cu) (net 17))
 (segment (start 132.0247 134.62) (end 127.2853 139.3594) (width 0.25) (layer B.Cu) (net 17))
 (segment (start 127.2853 139.3594) (end 121.3053 139.3594) (width 0.25) (layer B.Cu) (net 17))
 (segment (start 121.3053 139.3594) (end 121.3053 146.05) (width 0.25) (layer B.Cu) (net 17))
 (segment (start 107.95 129.54) (end 109.0753 129.54) (width 0.25) (layer B.Cu) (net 17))
 (segment (start 133.35 134.62) (end 132.0247 134.62) (width 0.25) (layer B.Cu) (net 17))
 (segment (start 119.38 146.05) (end 121.3053 146.05) (width 0.25) (layer B.Cu) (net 17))
 (segment (start 134.0127 134.62) (end 133.35 134.62) (width 0.25) (layer B.Cu) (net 17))
 (segment (start 134.0127 134.62) (end 134.6753 134.62) (width 0.25) (layer B.Cu) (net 17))
 (segment (start 134.6753 134.62) (end 135.9453 133.35) (width 0.25) (layer B.Cu) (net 17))
 (segment (start 135.9453 133.35) (end 143.51 133.35) (width 0.25) (layer B.Cu) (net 17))
 (segment (start 121.3644 149.42) (end 106.3253 149.42) (width 0.25) (layer F.Cu) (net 2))
 (segment (start 106.3253 149.42) (end 105.8653 149.88) (width 0.25) (layer F.Cu) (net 2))
 (segment (start 125.73 149.86) (end 125.29 149.42) (width 0.25) (layer F.Cu) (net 2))
 (segment (start 125.29 149.42) (end 121.3644 149.42) (width 0.25) (layer F.Cu) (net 2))
 (segment (start 119.38 132.7353) (end 121.3644 134.7197) (width 0.25) (layer F.Cu) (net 2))
 (segment (start 121.3644 134.7197) (end 121.3644 149.42) (width 0.25) (layer F.Cu) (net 2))
 (segment (start 104.14 149.88) (end 105.8653 149.88) (width 0.25) (layer F.Cu) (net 2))
 (segment (start 119.38 130.81) (end 119.38 132.7353) (width 0.25) (layer F.Cu) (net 2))
 (segment (start 104.14 144.78) (end 102.4147 144.78) (width 0.25) (layer B.Cu) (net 5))
 (segment (start 97.79 151.13) (end 97.79 150.0047) (width 0.25) (layer B.Cu) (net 5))
 (segment (start 97.79 150.0047) (end 102.4147 145.38) (width 0.25) (layer B.Cu) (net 5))
 (segment (start 102.4147 145.38) (end 102.4147 144.78) (width 0.25) (layer B.Cu) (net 5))
 (segment (start 105.8653 139.7) (end 102.87 139.7) (width 0.25) (layer B.Cu) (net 4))
 (segment (start 107.95 139.7) (end 105.8653 139.7) (width 0.25) (layer B.Cu) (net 4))
 (segment (start 105.8653 139.7) (end 105.8653 146.48) (width 0.25) (layer B.Cu) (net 4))
 (segment (start 104.14 146.48) (end 105.8653 146.48) (width 0.25) (layer B.Cu) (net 4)))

